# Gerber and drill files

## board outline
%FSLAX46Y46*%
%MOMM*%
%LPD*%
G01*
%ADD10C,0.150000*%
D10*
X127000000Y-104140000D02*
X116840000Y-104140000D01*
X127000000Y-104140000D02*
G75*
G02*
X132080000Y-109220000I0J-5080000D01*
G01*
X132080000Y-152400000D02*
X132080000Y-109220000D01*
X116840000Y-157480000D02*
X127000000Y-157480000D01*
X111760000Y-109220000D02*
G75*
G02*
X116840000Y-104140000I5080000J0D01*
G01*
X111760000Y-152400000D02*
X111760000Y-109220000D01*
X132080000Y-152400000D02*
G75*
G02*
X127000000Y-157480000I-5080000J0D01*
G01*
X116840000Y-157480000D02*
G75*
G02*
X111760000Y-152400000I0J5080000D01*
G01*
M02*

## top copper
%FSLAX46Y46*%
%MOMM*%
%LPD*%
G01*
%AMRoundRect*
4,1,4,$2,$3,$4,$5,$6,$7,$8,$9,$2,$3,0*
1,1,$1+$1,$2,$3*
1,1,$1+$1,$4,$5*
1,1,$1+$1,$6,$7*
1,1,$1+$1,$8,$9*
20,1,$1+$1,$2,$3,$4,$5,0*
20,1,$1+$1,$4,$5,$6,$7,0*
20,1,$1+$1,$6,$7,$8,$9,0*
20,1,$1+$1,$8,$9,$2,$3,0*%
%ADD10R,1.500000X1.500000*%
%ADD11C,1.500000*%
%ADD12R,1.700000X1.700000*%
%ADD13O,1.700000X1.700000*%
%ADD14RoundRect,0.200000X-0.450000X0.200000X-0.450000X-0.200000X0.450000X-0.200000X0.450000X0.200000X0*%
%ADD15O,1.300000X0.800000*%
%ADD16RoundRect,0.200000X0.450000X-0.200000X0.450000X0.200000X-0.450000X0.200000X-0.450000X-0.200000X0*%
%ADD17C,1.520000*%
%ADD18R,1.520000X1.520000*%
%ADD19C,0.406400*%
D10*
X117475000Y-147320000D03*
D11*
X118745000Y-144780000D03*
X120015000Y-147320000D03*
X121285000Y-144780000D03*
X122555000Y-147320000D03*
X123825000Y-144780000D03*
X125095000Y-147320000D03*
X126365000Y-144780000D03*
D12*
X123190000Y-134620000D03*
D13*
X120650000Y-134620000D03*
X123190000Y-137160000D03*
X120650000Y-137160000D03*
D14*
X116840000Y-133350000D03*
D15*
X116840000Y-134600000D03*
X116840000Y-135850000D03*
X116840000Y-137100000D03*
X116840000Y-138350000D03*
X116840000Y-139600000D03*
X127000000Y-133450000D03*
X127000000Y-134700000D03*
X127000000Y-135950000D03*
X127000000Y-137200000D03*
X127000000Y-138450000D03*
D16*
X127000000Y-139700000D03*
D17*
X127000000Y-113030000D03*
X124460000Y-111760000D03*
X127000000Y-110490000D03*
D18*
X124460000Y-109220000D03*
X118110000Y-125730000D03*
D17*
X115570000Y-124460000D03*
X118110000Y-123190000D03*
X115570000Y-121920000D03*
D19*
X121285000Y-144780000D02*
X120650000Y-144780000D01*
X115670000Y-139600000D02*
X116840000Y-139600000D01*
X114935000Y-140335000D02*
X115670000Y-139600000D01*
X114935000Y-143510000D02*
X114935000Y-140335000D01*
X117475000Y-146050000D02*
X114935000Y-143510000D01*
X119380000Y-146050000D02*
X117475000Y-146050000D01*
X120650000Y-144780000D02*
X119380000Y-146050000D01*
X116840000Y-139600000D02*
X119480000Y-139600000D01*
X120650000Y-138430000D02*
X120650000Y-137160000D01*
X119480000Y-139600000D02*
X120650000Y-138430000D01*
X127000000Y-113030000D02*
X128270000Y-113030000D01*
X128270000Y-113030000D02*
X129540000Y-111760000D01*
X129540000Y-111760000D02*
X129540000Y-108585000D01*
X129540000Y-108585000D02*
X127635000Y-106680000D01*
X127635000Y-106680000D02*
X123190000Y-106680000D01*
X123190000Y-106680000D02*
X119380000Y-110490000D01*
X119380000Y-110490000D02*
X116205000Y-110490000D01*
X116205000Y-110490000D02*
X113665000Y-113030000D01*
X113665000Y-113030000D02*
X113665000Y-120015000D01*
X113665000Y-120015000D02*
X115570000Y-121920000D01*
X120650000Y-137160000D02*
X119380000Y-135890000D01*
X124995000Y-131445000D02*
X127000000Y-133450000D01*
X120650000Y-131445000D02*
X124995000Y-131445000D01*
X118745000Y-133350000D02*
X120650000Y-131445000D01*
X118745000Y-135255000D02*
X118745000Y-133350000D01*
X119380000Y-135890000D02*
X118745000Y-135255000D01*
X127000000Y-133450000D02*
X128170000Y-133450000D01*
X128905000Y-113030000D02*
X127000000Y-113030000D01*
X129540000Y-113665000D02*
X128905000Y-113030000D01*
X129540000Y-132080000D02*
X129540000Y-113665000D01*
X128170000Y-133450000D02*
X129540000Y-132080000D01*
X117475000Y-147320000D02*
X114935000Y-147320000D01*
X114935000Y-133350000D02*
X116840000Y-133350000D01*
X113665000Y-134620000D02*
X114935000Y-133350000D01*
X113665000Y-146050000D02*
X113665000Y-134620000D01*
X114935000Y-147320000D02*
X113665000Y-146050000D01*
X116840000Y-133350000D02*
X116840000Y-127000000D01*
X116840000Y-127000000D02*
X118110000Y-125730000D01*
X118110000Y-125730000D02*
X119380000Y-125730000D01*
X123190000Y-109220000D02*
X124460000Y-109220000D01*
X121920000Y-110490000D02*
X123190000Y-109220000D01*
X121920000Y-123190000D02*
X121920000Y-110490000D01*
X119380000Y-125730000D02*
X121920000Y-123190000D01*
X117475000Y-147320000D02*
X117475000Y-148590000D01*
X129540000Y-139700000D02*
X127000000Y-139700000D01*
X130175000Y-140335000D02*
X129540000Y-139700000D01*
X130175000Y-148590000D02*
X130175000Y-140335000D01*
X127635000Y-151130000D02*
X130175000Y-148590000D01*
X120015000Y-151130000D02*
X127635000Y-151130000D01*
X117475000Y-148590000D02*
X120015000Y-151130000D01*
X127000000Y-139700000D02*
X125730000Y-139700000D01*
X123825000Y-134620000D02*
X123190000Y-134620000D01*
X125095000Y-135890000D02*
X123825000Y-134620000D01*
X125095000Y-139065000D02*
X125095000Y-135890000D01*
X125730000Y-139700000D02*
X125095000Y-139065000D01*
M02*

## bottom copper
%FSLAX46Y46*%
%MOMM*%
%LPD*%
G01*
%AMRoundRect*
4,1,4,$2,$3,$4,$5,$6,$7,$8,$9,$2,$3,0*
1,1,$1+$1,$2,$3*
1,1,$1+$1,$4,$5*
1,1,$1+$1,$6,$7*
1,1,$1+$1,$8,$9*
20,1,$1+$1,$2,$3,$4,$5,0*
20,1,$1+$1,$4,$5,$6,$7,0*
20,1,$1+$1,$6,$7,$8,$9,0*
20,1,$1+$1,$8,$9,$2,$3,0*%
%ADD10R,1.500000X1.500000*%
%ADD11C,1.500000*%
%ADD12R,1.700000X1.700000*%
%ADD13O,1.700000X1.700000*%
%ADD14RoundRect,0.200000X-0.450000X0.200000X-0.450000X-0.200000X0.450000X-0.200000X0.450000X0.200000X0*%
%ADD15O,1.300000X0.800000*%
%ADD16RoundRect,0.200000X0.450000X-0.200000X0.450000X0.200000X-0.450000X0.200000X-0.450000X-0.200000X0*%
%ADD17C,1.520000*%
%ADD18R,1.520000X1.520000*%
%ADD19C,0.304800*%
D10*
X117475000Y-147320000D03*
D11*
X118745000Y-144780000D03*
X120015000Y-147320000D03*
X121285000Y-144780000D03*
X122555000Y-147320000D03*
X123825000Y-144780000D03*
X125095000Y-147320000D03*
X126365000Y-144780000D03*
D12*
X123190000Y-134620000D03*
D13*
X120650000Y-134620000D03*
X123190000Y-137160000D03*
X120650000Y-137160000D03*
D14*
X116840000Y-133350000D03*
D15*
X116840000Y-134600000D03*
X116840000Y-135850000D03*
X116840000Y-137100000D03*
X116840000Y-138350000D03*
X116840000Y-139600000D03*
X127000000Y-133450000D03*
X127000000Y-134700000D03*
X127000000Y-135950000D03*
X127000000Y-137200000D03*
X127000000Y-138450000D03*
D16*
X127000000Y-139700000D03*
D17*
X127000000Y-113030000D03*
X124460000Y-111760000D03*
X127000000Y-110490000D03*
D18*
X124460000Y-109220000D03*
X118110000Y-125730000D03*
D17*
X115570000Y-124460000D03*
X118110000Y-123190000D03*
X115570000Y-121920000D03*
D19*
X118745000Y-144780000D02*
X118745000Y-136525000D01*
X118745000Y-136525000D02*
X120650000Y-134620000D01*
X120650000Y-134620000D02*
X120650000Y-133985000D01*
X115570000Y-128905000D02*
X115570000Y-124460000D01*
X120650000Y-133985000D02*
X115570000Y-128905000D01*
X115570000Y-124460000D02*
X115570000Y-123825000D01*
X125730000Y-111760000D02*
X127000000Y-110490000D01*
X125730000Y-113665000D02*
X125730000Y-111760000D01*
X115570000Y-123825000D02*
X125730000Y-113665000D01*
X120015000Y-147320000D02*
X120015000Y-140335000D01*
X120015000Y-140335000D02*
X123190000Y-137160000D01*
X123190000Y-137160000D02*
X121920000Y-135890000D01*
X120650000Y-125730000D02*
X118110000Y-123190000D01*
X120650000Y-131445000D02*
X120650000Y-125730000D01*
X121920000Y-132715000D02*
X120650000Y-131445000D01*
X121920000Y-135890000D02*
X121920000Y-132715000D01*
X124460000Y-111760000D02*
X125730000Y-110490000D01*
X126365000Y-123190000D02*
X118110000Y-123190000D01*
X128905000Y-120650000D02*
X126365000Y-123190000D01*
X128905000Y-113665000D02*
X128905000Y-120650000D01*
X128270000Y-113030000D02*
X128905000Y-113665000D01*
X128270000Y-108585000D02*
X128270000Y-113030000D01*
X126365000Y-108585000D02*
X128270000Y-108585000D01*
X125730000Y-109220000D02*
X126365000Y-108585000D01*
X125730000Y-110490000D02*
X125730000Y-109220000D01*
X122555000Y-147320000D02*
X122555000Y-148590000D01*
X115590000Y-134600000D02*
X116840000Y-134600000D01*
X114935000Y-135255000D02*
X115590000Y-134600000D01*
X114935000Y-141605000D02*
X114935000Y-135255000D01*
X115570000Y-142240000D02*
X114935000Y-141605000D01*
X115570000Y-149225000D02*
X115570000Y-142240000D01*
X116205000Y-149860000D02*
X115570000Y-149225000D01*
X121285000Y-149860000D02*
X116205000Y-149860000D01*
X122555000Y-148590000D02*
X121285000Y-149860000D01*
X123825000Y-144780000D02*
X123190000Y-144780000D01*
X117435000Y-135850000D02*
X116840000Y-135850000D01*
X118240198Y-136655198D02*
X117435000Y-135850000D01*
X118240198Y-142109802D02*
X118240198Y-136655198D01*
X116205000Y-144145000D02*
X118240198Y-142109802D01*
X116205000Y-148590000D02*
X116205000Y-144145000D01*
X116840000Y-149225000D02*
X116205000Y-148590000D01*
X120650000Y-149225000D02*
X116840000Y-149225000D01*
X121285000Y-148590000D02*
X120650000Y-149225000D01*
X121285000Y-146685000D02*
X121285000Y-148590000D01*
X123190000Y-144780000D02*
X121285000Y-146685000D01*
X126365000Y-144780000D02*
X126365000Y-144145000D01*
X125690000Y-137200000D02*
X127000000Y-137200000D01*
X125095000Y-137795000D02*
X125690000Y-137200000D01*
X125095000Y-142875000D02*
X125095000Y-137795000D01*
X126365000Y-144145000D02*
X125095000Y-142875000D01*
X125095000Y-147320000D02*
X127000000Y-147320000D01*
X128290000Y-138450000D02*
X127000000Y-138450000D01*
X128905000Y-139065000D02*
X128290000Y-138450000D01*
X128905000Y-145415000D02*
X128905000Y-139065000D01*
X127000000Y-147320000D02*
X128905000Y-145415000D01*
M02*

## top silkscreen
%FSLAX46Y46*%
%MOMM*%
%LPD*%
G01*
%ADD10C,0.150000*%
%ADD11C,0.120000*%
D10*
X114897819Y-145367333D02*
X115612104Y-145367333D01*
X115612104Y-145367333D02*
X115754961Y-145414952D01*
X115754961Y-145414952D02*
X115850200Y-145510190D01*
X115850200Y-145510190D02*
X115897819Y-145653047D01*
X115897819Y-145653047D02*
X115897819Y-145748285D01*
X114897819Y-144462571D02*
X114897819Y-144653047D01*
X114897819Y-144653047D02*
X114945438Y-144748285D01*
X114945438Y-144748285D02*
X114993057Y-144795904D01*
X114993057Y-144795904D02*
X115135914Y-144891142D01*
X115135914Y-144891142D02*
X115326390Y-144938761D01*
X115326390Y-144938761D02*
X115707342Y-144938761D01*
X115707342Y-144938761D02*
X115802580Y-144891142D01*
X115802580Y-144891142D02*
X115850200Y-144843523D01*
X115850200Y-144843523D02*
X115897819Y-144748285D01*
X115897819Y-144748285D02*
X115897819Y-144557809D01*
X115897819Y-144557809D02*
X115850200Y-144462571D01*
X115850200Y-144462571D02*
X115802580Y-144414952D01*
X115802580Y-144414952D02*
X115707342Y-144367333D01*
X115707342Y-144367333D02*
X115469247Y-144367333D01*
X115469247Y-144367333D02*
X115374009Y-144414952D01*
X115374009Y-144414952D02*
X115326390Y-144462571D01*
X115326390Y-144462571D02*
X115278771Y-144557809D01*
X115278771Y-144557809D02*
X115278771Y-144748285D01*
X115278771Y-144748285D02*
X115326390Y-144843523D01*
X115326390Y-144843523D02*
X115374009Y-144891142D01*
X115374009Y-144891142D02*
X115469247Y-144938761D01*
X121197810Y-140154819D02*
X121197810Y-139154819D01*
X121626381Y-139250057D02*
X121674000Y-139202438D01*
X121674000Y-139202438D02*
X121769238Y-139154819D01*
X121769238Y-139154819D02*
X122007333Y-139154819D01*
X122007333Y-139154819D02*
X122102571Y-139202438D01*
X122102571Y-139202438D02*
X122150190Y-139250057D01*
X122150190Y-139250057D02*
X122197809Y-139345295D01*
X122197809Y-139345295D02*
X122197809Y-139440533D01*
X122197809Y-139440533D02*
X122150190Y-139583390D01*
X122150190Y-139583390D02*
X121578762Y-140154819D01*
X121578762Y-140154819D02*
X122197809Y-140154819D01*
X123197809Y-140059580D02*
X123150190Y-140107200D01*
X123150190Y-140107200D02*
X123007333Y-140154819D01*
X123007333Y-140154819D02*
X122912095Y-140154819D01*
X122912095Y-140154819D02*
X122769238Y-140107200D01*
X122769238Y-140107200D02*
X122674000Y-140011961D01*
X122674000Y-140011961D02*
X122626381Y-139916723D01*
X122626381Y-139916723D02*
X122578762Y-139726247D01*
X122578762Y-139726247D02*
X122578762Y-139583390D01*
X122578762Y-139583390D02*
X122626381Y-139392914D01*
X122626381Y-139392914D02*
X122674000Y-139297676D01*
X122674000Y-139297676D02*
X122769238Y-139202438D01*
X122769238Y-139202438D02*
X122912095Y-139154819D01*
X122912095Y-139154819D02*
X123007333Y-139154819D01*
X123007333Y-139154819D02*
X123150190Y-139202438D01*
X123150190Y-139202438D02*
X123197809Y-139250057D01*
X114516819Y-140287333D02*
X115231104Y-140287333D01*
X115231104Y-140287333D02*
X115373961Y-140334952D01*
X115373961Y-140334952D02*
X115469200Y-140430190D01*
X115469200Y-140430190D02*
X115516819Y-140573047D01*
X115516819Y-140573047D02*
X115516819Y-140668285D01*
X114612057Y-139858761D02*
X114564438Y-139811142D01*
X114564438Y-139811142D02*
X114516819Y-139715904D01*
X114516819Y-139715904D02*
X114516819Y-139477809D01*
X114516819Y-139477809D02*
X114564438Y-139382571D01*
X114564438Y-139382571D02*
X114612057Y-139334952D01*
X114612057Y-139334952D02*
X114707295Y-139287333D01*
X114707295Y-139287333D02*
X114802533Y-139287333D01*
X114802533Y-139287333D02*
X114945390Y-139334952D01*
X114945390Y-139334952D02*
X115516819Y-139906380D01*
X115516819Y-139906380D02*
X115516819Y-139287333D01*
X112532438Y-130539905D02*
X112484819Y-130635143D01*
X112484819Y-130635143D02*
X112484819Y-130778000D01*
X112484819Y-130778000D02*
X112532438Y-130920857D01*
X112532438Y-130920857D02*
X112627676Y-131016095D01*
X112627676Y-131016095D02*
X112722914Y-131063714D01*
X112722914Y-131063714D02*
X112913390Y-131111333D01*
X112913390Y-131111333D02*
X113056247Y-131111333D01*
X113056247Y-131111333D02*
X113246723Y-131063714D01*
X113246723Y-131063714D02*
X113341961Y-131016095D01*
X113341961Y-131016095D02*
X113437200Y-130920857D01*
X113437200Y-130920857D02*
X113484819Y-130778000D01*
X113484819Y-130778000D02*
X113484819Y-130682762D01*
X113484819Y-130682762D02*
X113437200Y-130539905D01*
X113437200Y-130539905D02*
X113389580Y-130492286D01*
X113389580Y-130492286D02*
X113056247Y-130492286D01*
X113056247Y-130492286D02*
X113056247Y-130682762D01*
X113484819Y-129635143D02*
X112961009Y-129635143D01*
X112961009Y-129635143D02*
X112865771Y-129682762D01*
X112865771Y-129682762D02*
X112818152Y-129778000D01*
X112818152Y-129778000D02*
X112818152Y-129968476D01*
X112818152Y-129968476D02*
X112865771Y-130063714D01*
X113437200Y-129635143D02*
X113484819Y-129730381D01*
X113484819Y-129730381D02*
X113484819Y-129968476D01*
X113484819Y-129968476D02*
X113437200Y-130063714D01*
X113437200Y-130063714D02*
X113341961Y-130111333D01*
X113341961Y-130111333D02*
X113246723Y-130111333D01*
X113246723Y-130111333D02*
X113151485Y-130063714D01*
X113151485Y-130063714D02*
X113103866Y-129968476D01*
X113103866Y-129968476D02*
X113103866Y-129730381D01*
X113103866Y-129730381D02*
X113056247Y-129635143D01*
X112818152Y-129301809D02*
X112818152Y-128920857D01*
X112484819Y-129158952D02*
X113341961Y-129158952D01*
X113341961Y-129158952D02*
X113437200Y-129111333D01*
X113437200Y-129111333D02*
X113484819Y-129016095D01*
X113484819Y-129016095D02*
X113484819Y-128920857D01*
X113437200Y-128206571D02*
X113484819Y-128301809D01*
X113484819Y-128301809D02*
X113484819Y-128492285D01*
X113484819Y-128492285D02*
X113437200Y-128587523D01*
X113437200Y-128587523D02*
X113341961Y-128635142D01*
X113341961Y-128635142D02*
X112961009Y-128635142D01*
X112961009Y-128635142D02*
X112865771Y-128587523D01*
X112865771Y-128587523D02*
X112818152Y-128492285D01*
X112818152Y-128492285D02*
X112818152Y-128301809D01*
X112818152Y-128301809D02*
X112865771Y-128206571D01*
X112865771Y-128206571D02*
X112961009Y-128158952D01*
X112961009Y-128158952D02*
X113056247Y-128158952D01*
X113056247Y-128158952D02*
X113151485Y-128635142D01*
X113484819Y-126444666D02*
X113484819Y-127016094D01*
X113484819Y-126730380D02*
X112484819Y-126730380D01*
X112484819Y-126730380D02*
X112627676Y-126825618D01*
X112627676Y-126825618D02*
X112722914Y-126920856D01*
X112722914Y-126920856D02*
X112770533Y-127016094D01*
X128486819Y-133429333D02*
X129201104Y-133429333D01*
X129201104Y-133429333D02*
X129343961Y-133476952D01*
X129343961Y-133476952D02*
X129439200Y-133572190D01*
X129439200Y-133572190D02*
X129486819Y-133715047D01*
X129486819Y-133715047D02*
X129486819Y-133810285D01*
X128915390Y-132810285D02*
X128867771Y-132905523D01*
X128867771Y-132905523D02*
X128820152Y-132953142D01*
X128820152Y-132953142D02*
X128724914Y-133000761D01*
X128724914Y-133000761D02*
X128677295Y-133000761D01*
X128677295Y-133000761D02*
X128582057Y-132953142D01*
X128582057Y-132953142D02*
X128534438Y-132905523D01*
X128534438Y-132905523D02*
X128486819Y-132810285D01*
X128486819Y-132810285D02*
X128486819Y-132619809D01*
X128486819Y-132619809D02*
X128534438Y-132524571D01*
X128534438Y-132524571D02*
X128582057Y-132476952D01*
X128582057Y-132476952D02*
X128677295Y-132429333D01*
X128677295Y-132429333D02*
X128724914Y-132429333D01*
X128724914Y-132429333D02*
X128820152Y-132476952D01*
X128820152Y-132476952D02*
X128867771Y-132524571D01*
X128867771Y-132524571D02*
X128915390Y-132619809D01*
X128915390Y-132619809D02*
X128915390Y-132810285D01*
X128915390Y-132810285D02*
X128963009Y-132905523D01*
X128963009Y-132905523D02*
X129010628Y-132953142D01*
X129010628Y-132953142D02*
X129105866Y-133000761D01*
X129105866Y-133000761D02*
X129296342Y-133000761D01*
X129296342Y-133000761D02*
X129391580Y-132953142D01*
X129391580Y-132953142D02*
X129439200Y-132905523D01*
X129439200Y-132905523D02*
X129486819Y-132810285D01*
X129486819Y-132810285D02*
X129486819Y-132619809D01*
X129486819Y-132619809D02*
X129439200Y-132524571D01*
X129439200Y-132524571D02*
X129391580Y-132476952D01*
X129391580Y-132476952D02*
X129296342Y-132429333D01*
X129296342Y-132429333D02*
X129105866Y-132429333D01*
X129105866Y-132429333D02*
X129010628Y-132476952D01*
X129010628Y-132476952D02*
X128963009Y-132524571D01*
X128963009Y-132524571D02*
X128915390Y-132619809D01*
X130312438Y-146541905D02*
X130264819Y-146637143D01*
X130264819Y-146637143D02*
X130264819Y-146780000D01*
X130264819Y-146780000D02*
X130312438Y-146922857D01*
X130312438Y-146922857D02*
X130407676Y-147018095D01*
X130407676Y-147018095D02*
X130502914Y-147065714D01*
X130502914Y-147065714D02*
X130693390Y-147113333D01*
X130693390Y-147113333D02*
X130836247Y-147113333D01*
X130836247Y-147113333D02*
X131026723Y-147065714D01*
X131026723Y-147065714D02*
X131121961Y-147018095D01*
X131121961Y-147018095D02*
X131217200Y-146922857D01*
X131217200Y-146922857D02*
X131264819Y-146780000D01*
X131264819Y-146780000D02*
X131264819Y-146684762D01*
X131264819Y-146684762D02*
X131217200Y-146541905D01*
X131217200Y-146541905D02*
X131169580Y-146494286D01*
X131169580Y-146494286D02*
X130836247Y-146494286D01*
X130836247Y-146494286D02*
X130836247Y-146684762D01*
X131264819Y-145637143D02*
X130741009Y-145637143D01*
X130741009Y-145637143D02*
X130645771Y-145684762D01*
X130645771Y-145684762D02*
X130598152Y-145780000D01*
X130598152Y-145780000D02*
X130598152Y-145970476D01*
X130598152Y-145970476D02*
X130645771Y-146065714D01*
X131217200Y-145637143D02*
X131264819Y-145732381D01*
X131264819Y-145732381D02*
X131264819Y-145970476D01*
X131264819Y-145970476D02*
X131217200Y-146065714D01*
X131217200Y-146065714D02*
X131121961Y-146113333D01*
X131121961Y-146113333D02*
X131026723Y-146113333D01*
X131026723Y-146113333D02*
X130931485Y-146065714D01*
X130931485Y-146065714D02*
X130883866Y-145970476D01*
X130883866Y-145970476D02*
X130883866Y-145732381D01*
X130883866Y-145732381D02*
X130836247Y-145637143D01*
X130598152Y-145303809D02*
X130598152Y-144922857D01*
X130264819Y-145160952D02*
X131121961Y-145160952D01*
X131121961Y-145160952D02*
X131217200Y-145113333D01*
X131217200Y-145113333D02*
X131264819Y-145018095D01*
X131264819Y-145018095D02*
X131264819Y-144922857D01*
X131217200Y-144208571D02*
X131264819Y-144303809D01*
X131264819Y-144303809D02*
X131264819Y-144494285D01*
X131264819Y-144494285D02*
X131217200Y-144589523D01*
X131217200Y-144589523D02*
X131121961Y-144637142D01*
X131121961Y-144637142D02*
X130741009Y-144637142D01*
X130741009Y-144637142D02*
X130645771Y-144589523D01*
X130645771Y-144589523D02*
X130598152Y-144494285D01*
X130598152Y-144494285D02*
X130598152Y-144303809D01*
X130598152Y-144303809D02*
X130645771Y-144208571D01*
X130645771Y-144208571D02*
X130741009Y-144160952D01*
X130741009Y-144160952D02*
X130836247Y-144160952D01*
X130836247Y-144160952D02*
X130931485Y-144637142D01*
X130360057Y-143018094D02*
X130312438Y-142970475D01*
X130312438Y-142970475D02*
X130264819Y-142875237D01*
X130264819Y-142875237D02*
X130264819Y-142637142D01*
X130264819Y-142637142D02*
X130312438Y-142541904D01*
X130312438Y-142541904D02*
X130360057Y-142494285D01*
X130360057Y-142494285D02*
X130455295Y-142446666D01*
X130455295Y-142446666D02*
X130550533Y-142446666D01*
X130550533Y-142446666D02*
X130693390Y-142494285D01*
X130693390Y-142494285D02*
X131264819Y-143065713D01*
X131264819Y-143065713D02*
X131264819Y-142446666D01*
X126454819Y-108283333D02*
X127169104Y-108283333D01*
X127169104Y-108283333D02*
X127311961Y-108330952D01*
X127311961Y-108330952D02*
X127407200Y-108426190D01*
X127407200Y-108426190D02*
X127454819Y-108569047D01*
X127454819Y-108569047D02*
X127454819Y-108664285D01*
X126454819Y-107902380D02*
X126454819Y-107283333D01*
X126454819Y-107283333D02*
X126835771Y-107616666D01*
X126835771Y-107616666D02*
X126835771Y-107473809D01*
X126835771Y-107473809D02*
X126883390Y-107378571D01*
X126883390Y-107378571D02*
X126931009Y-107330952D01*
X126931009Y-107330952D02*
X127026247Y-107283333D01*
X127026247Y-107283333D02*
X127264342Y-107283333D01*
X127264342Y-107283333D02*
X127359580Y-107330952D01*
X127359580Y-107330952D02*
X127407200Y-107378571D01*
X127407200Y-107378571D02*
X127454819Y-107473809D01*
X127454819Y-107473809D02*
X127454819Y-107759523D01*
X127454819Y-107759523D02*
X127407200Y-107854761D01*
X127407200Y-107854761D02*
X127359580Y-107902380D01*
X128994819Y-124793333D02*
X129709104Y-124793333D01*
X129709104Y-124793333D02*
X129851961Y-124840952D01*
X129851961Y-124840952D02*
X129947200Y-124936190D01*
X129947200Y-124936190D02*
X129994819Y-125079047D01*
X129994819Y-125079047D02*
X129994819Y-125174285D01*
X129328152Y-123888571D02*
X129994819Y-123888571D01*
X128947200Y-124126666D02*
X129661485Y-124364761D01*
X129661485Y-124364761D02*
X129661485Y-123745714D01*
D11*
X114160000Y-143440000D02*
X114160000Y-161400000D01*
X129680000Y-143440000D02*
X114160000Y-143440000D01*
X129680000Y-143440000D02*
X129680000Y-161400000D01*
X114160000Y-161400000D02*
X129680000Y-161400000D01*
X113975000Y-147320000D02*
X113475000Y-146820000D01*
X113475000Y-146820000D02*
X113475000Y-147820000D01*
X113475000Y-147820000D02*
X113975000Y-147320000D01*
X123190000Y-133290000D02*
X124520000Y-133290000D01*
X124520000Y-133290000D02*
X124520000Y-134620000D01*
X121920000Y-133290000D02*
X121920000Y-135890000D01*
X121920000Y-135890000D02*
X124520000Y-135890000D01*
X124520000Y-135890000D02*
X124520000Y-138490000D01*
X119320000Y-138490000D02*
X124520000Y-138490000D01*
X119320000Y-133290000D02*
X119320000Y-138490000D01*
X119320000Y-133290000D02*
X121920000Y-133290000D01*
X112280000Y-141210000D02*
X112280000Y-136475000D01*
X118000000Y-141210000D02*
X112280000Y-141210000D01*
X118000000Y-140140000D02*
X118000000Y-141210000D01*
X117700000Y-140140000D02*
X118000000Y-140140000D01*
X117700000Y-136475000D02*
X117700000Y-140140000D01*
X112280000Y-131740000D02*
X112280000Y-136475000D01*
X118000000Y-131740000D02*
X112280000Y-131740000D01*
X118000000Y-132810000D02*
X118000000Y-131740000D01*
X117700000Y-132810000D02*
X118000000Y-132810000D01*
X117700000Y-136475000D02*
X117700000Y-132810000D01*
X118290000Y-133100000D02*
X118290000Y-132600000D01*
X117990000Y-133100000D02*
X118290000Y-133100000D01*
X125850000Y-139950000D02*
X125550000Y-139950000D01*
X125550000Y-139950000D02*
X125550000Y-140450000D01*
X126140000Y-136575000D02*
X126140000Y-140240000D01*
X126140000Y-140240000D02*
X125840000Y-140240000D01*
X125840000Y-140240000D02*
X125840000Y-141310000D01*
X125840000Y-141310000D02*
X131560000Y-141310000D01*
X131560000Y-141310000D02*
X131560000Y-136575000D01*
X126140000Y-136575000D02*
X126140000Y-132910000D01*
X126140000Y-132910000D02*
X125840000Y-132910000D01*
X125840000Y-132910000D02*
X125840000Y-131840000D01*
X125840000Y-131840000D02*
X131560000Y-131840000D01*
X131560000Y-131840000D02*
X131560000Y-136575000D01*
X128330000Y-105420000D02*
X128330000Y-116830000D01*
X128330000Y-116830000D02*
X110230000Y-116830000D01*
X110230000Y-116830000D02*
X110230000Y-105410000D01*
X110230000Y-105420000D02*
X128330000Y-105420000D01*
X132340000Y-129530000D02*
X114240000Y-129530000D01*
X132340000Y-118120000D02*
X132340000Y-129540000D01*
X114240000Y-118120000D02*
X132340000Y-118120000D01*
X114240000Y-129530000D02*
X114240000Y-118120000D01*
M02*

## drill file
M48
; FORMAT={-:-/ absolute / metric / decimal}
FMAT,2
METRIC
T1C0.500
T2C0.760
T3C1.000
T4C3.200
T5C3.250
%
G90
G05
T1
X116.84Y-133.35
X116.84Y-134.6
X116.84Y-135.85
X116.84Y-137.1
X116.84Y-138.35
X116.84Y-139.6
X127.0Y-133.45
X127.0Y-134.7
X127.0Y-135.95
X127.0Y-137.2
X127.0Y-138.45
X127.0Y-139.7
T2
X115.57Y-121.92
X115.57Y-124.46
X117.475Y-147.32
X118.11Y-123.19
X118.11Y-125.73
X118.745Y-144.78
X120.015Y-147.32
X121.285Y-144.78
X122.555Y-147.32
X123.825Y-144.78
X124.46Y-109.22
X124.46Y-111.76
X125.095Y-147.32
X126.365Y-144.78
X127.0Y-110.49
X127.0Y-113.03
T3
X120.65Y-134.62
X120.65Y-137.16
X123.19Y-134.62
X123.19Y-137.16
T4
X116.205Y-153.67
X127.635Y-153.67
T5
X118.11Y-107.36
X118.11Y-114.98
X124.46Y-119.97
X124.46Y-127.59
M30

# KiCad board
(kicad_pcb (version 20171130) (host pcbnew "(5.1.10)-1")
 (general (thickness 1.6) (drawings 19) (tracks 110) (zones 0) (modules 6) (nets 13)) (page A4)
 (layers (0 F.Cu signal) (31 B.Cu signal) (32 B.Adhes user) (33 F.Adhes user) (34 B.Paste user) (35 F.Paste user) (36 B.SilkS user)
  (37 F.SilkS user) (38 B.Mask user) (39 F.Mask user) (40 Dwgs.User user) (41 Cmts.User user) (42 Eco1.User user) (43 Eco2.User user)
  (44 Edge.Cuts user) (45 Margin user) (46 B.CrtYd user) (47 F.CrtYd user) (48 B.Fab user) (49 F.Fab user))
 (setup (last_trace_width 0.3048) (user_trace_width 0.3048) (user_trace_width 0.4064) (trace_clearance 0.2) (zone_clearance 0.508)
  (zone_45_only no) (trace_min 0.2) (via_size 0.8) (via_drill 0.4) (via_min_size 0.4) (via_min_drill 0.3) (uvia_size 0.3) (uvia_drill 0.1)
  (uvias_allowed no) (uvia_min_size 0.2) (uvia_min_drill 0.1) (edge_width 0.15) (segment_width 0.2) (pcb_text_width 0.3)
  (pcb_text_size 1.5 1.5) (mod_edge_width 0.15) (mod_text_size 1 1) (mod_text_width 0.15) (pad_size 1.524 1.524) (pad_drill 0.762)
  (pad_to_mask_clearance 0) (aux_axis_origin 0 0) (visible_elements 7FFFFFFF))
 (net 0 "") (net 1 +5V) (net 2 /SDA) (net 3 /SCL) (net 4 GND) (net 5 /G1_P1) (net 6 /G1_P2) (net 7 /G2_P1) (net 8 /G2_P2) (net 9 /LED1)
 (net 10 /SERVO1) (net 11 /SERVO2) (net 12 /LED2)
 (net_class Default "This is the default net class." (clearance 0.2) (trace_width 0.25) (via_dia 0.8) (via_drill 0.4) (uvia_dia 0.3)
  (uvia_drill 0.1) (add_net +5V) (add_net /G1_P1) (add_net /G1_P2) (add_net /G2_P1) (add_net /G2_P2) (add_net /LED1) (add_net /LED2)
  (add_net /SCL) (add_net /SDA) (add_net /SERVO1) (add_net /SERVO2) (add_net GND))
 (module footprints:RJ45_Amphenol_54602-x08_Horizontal (layer F.Cu) (at 117.475 147.32)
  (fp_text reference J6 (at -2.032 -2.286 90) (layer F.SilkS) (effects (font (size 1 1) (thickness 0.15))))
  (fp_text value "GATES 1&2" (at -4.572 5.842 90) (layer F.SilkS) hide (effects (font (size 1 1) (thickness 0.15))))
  (fp_line (start -3.315 -3.88) (end -3.315 14.08) (layer F.SilkS) (width 0.12))
  (fp_line (start 12.205 -3.88) (end -3.315 -3.88) (layer F.SilkS) (width 0.12))
  (fp_line (start 12.205 -3.88) (end 12.205 14.08) (layer F.SilkS) (width 0.12))
  (fp_line (start -3.315 14.08) (end 12.205 14.08) (layer F.SilkS) (width 0.12))
  (fp_line (start -3.5 0) (end -4 -0.5) (layer F.SilkS) (width 0.12))
  (fp_line (start -4 -0.5) (end -4 0.5) (layer F.SilkS) (width 0.12))
  (fp_line (start -4 0.5) (end -3.5 0) (layer F.SilkS) (width 0.12))
  (pad "" np_thru_hole circle (at 10.16 6.35) (size 3.2 3.2) (drill 3.2) (layers *.Cu *.Mask))
  (pad "" np_thru_hole circle (at -1.27 6.35) (size 3.2 3.2) (drill 3.2) (layers *.Cu *.Mask))
  (pad 1 thru_hole rect (at 0 0) (size 1.5 1.5) (drill 0.76) (layers *.Cu *.Mask) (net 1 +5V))
  (pad 2 thru_hole circle (at 1.27 -2.54) (size 1.5 1.5) (drill 0.76) (layers *.Cu *.Mask) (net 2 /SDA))
  (pad 3 thru_hole circle (at 2.54 0) (size 1.5 1.5) (drill 0.76) (layers *.Cu *.Mask) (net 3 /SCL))
  (pad 4 thru_hole circle (at 3.81 -2.54) (size 1.5 1.5) (drill 0.76) (layers *.Cu *.Mask) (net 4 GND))
  (pad 5 thru_hole circle (at 5.08 0) (size 1.5 1.5) (drill 0.76) (layers *.Cu *.Mask) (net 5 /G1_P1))
  (pad 6 thru_hole circle (at 6.35 -2.54) (size 1.5 1.5) (drill 0.76) (layers *.Cu *.Mask) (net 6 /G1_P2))
  (pad 7 thru_hole circle (at 7.62 0) (size 1.5 1.5) (drill 0.76) (layers *.Cu *.Mask) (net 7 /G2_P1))
  (pad 8 thru_hole circle (at 8.89 -2.54) (size 1.5 1.5) (drill 0.76) (layers *.Cu *.Mask) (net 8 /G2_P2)))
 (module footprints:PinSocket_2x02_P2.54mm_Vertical (layer F.Cu) (at 123.19 134.62)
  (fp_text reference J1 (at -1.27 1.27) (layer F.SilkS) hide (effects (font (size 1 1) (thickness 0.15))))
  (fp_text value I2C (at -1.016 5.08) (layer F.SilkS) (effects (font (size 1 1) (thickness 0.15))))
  (fp_line (start 0 -1.33) (end 1.33 -1.33) (layer F.SilkS) (width 0.12))
  (fp_line (start 1.33 -1.33) (end 1.33 0) (layer F.SilkS) (width 0.12))
  (fp_line (start -1.27 -1.33) (end -1.27 1.27) (layer F.SilkS) (width 0.12))
  (fp_line (start -1.27 1.27) (end 1.33 1.27) (layer F.SilkS) (width 0.12))
  (fp_line (start 1.33 1.27) (end 1.33 3.87) (layer F.SilkS) (width 0.12))
  (fp_line (start -3.87 3.87) (end 1.33 3.87) (layer F.SilkS) (width 0.12))
  (fp_line (start -3.87 -1.33) (end -3.87 3.87) (layer F.SilkS) (width 0.12))
  (fp_line (start -3.87 -1.33) (end -1.27 -1.33) (layer F.SilkS) (width 0.12))
  (pad 1 thru_hole rect (at 0 0) (size 1.7 1.7) (drill 1) (layers *.Cu *.Mask) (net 1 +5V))
  (pad 2 thru_hole oval (at -2.54 0) (size 1.7 1.7) (drill 1) (layers *.Cu *.Mask) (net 2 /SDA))
  (pad 3 thru_hole oval (at 0 2.54) (size 1.7 1.7) (drill 1) (layers *.Cu *.Mask) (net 3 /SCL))
  (pad 4 thru_hole oval (at -2.54 2.54) (size 1.7 1.7) (drill 1) (layers *.Cu *.Mask) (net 4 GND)))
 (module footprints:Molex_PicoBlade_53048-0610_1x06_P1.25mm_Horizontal (layer F.Cu) (at 116.84 133.35 270)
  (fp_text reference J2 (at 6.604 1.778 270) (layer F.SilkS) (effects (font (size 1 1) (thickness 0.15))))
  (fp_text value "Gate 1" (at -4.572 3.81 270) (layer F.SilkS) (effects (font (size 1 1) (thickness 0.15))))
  (fp_line (start 7.86 4.56) (end 3.125 4.56) (layer F.SilkS) (width 0.12))
  (fp_line (start 7.86 -1.16) (end 7.86 4.56) (layer F.SilkS) (width 0.12))
  (fp_line (start 6.79 -1.16) (end 7.86 -1.16) (layer F.SilkS) (width 0.12))
  (fp_line (start 6.79 -0.86) (end 6.79 -1.16) (layer F.SilkS) (width 0.12))
  (fp_line (start 3.125 -0.86) (end 6.79 -0.86) (layer F.SilkS) (width 0.12))
  (fp_line (start -1.61 4.56) (end 3.125 4.56) (layer F.SilkS) (width 0.12))
  (fp_line (start -1.61 -1.16) (end -1.61 4.56) (layer F.SilkS) (width 0.12))
  (fp_line (start -0.54 -1.16) (end -1.61 -1.16) (layer F.SilkS) (width 0.12))
  (fp_line (start -0.54 -0.86) (end -0.54 -1.16) (layer F.SilkS) (width 0.12))
  (fp_line (start 3.125 -0.86) (end -0.54 -0.86) (layer F.SilkS) (width 0.12))
  (fp_line (start -0.25 -1.45) (end -0.75 -1.45) (layer F.SilkS) (width 0.12))
  (fp_line (start -0.25 -1.15) (end -0.25 -1.45) (layer F.SilkS) (width 0.12))
  (pad 1 thru_hole roundrect (at 0 0 270) (size 0.8 1.3) (drill 0.5) (layers *.Cu *.Mask) (roundrect_rratio 0.25) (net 1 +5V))
  (pad 2 thru_hole oval (at 1.25 0 270) (size 0.8 1.3) (drill 0.5) (layers *.Cu *.Mask) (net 5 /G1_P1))
  (pad 3 thru_hole oval (at 2.5 0 270) (size 0.8 1.3) (drill 0.5) (layers *.Cu *.Mask) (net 6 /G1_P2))
  (pad 4 thru_hole oval (at 3.75 0 270) (size 0.8 1.3) (drill 0.5) (layers *.Cu *.Mask) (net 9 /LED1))
  (pad 5 thru_hole oval (at 5 0 270) (size 0.8 1.3) (drill 0.5) (layers *.Cu *.Mask) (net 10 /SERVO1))
  (pad 6 thru_hole oval (at 6.25 0 270) (size 0.8 1.3) (drill 0.5) (layers *.Cu *.Mask) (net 4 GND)))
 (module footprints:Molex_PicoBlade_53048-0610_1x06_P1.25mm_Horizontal (layer F.Cu) (at 127 139.7 90)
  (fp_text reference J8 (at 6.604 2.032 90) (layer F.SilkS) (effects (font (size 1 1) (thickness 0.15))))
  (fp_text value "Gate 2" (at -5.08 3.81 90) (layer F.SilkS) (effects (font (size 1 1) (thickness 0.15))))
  (fp_line (start -0.25 -1.15) (end -0.25 -1.45) (layer F.SilkS) (width 0.12))
  (fp_line (start -0.25 -1.45) (end -0.75 -1.45) (layer F.SilkS) (width 0.12))
  (fp_line (start 3.125 -0.86) (end -0.54 -0.86) (layer F.SilkS) (width 0.12))
  (fp_line (start -0.54 -0.86) (end -0.54 -1.16) (layer F.SilkS) (width 0.12))
  (fp_line (start -0.54 -1.16) (end -1.61 -1.16) (layer F.SilkS) (width 0.12))
  (fp_line (start -1.61 -1.16) (end -1.61 4.56) (layer F.SilkS) (width 0.12))
  (fp_line (start -1.61 4.56) (end 3.125 4.56) (layer F.SilkS) (width 0.12))
  (fp_line (start 3.125 -0.86) (end 6.79 -0.86) (layer F.SilkS) (width 0.12))
  (fp_line (start 6.79 -0.86) (end 6.79 -1.16) (layer F.SilkS) (width 0.12))
  (fp_line (start 6.79 -1.16) (end 7.86 -1.16) (layer F.SilkS) (width 0.12))
  (fp_line (start 7.86 -1.16) (end 7.86 4.56) (layer F.SilkS) (width 0.12))
  (fp_line (start 7.86 4.56) (end 3.125 4.56) (layer F.SilkS) (width 0.12))
  (pad 6 thru_hole oval (at 6.25 0 90) (size 0.8 1.3) (drill 0.5) (layers *.Cu *.Mask) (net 4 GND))
  (pad 5 thru_hole oval (at 5 0 90) (size 0.8 1.3) (drill 0.5) (layers *.Cu *.Mask) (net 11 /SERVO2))
  (pad 4 thru_hole oval (at 3.75 0 90) (size 0.8 1.3) (drill 0.5) (layers *.Cu *.Mask) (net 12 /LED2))
  (pad 3 thru_hole oval (at 2.5 0 90) (size 0.8 1.3) (drill 0.5) (layers *.Cu *.Mask) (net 8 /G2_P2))
  (pad 2 thru_hole oval (at 1.25 0 90) (size 0.8 1.3) (drill 0.5) (layers *.Cu *.Mask) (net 7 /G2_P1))
  (pad 1 thru_hole roundrect (at 0 0 90) (size 0.8 1.3) (drill 0.5) (layers *.Cu *.Mask) (roundrect_rratio 0.25) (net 1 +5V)))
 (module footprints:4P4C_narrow (layer F.Cu) (at 127 109.22 270)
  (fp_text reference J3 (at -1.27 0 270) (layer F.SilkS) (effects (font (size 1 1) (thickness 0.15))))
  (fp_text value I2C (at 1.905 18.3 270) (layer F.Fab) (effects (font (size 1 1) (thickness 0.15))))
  (fp_line (start -3.8 -1.33) (end 7.61 -1.33) (layer F.SilkS) (width 0.12))
  (fp_line (start 7.61 -1.33) (end 7.61 16.77) (layer F.SilkS) (width 0.12))
  (fp_line (start 7.61 16.77) (end -3.81 16.77) (layer F.SilkS) (width 0.12))
  (fp_line (start -3.8 16.77) (end -3.8 -1.33) (layer F.SilkS) (width 0.12))
  (pad "" np_thru_hole circle (at 5.76 8.89 270) (size 3.25 3.25) (drill 3.25) (layers *.Cu *.Mask))
  (pad 4 thru_hole circle (at 3.81 0 270) (size 1.52 1.52) (drill 0.76) (layers *.Cu *.Mask) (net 4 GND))
  (pad 3 thru_hole circle (at 2.54 2.54 270) (size 1.52 1.52) (drill 0.76) (layers *.Cu *.Mask) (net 3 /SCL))
  (pad 2 thru_hole circle (at 1.27 0 270) (size 1.52 1.52) (drill 0.76) (layers *.Cu *.Mask) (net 2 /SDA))
  (pad "" np_thru_hole circle (at -1.86 8.89 270) (size 3.25 3.25) (drill 3.25) (layers *.Cu *.Mask))
  (pad 1 thru_hole rect (at 0 2.54 270) (size 1.52 1.52) (drill 0.76) (layers *.Cu *.Mask) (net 1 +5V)))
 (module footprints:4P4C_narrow (layer F.Cu) (at 115.57 125.73 90)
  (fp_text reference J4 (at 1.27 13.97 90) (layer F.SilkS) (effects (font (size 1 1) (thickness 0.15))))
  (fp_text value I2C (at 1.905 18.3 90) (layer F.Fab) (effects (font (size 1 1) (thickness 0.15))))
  (fp_line (start -3.8 16.77) (end -3.8 -1.33) (layer F.SilkS) (width 0.12))
  (fp_line (start 7.61 16.77) (end -3.81 16.77) (layer F.SilkS) (width 0.12))
  (fp_line (start 7.61 -1.33) (end 7.61 16.77) (layer F.SilkS) (width 0.12))
  (fp_line (start -3.8 -1.33) (end 7.61 -1.33) (layer F.SilkS) (width 0.12))
  (pad 1 thru_hole rect (at 0 2.54 90) (size 1.52 1.52) (drill 0.76) (layers *.Cu *.Mask) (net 1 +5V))
  (pad "" np_thru_hole circle (at -1.86 8.89 90) (size 3.25 3.25) (drill 3.25) (layers *.Cu *.Mask))
  (pad 2 thru_hole circle (at 1.27 0 90) (size 1.52 1.52) (drill 0.76) (layers *.Cu *.Mask) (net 2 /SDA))
  (pad 3 thru_hole circle (at 2.54 2.54 90) (size 1.52 1.52) (drill 0.76) (layers *.Cu *.Mask) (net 3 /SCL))
  (pad 4 thru_hole circle (at 3.81 0 90) (size 1.52 1.52) (drill 0.76) (layers *.Cu *.Mask) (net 4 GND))
  (pad "" np_thru_hole circle (at 5.76 8.89 90) (size 3.25 3.25) (drill 3.25) (layers *.Cu *.Mask)))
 (gr_line (start 127 104.14) (end 116.84 104.14) (angle 90) (layer Edge.Cuts) (width 0.15))
 (gr_arc (start 127 109.22) (end 127 104.14) (angle 90) (layer Edge.Cuts) (width 0.15))
 (gr_line (start 132.08 152.4) (end 132.08 109.22) (angle 90) (layer Edge.Cuts) (width 0.15))
 (gr_line (start 116.84 157.48) (end 127 157.48) (angle 90) (layer Edge.Cuts) (width 0.15))
 (gr_arc (start 116.84 109.22) (end 111.76 109.22) (angle 90) (layer Edge.Cuts) (width 0.15))
 (gr_line (start 111.76 152.4) (end 111.76 109.22) (angle 90) (layer Edge.Cuts) (width 0.15))
 (gr_arc (start 127 152.4) (end 132.08 152.4) (angle 90) (layer Edge.Cuts) (width 0.15))
 (gr_arc (start 116.84 152.4) (end 116.84 157.48) (angle 90) (layer Edge.Cuts) (width 0.15))
 (segment (start 121.285 144.78) (end 120.65 144.78) (width 0.4064) (layer F.Cu) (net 4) (status C00000))
 (segment (start 115.67 139.6) (end 116.84 139.6) (width 0.4064) (layer F.Cu) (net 4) (status 800000))
 (segment (start 114.935 140.335) (end 115.67 139.6) (width 0.4064) (layer F.Cu) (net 4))
 (segment (start 114.935 143.51) (end 114.935 140.335) (width 0.4064) (layer F.Cu) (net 4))
 (segment (start 117.475 146.05) (end 114.935 143.51) (width 0.4064) (layer F.Cu) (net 4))
 (segment (start 119.38 146.05) (end 117.475 146.05) (width 0.4064) (layer F.Cu) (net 4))
 (segment (start 120.65 144.78) (end 119.38 146.05) (width 0.4064) (layer F.Cu) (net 4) (status 400000))
 (segment (start 116.84 139.6) (end 119.48 139.6) (width 0.4064) (layer F.Cu) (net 4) (status 400000))
 (segment (start 120.65 138.43) (end 120.65 137.16) (width 0.4064) (layer F.Cu) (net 4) (status 800000))
 (segment (start 119.48 139.6) (end 120.65 138.43) (width 0.4064) (layer F.Cu) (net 4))
 (segment (start 127 113.03) (end 128.27 113.03) (width 0.4064) (layer F.Cu) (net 4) (status 400000))
 (segment (start 128.27 113.03) (end 129.54 111.76) (width 0.4064) (layer F.Cu) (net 4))
 (segment (start 129.54 111.76) (end 129.54 108.585) (width 0.4064) (layer F.Cu) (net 4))
 (segment (start 129.54 108.585) (end 127.635 106.68) (width 0.4064) (layer F.Cu) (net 4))
 (segment (start 127.635 106.68) (end 123.19 106.68) (width 0.4064) (layer F.Cu) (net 4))
 (segment (start 123.19 106.68) (end 119.38 110.49) (width 0.4064) (layer F.Cu) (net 4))
 (segment (start 119.38 110.49) (end 116.205 110.49) (width 0.4064) (layer F.Cu) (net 4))
 (segment (start 116.205 110.49) (end 113.665 113.03) (width 0.4064) (layer F.Cu) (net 4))
 (segment (start 113.665 113.03) (end 113.665 120.015) (width 0.4064) (layer F.Cu) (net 4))
 (segment (start 113.665 120.015) (end 115.57 121.92) (width 0.4064) (layer F.Cu) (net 4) (status 800000))
 (segment (start 120.65 137.16) (end 119.38 135.89) (width 0.4064) (layer F.Cu) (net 4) (status 400000))
 (segment (start 124.995 131.445) (end 127 133.45) (width 0.4064) (layer F.Cu) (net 4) (status 800000))
 (segment (start 120.65 131.445) (end 124.995 131.445) (width 0.4064) (layer F.Cu) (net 4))
 (segment (start 118.745 133.35) (end 120.65 131.445) (width 0.4064) (layer F.Cu) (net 4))
 (segment (start 118.745 135.255) (end 118.745 133.35) (width 0.4064) (layer F.Cu) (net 4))
 (segment (start 119.38 135.89) (end 118.745 135.255) (width 0.4064) (layer F.Cu) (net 4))
 (segment (start 127 133.45) (end 128.17 133.45) (width 0.4064) (layer F.Cu) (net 4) (status 400000))
 (segment (start 128.905 113.03) (end 127 113.03) (width 0.4064) (layer F.Cu) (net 4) (status 800000))
 (segment (start 129.54 113.665) (end 128.905 113.03) (width 0.4064) (layer F.Cu) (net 4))
 (segment (start 129.54 132.08) (end 129.54 113.665) (width 0.4064) (layer F.Cu) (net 4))
 (segment (start 128.17 133.45) (end 129.54 132.08) (width 0.4064) (layer F.Cu) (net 4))
 (segment (start 118.745 144.78) (end 118.745 136.525) (width 0.3048) (layer B.Cu) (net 2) (status 400000))
 (segment (start 118.745 136.525) (end 120.65 134.62) (width 0.3048) (layer B.Cu) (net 2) (status 800000))
 (segment (start 120.65 134.62) (end 120.65 133.985) (width 0.3048) (layer B.Cu) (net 2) (status C00000))
 (segment (start 115.57 128.905) (end 115.57 124.46) (width 0.3048) (layer B.Cu) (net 2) (status 800000))
 (segment (start 120.65 133.985) (end 115.57 128.905) (width 0.3048) (layer B.Cu) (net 2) (status 400000))
 (segment (start 115.57 124.46) (end 115.57 123.825) (width 0.3048) (layer B.Cu) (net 2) (status C00000))
 (segment (start 125.73 111.76) (end 127 110.49) (width 0.3048) (layer B.Cu) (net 2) (status 800000))
 (segment (start 125.73 113.665) (end 125.73 111.76) (width 0.3048) (layer B.Cu) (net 2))
 (segment (start 115.57 123.825) (end 125.73 113.665) (width 0.3048) (layer B.Cu) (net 2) (status 400000))
 (segment (start 120.015 147.32) (end 120.015 140.335) (width 0.3048) (layer B.Cu) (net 3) (status 400000))
 (segment (start 120.015 140.335) (end 123.19 137.16) (width 0.3048) (layer B.Cu) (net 3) (status 800000))
 (segment (start 123.19 137.16) (end 121.92 135.89) (width 0.3048) (layer B.Cu) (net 3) (status 400000))
 (segment (start 120.65 125.73) (end 118.11 123.19) (width 0.3048) (layer B.Cu) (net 3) (status 800000))
 (segment (start 120.65 131.445) (end 120.65 125.73) (width 0.3048) (layer B.Cu) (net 3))
 (segment (start 121.92 132.715) (end 120.65 131.445) (width 0.3048) (layer B.Cu) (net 3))
 (segment (start 121.92 135.89) (end 121.92 132.715) (width 0.3048) (layer B.Cu) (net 3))
 (segment (start 124.46 111.76) (end 125.73 110.49) (width 0.3048) (layer B.Cu) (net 3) (status 400000))
 (segment (start 126.365 123.19) (end 118.11 123.19) (width 0.3048) (layer B.Cu) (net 3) (status 800000))
 (segment (start 128.905 120.65) (end 126.365 123.19) (width 0.3048) (layer B.Cu) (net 3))
 (segment (start 128.905 113.665) (end 128.905 120.65) (width 0.3048) (layer B.Cu) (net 3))
 (segment (start 128.27 113.03) (end 128.905 113.665) (width 0.3048) (layer B.Cu) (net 3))
 (segment (start 128.27 108.585) (end 128.27 113.03) (width 0.3048) (layer B.Cu) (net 3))
 (segment (start 126.365 108.585) (end 128.27 108.585) (width 0.3048) (layer B.Cu) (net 3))
 (segment (start 125.73 109.22) (end 126.365 108.585) (width 0.3048) (layer B.Cu) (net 3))
 (segment (start 125.73 110.49) (end 125.73 109.22) (width 0.3048) (layer B.Cu) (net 3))
 (segment (start 117.475 147.32) (end 114.935 147.32) (width 0.4064) (layer F.Cu) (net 1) (status 400000))
 (segment (start 114.935 133.35) (end 116.84 133.35) (width 0.4064) (layer F.Cu) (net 1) (status 800000))
 (segment (start 113.665 134.62) (end 114.935 133.35) (width 0.4064) (layer F.Cu) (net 1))
 (segment (start 113.665 146.05) (end 113.665 134.62) (width 0.4064) (layer F.Cu) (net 1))
 (segment (start 114.935 147.32) (end 113.665 146.05) (width 0.4064) (layer F.Cu) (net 1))
 (segment (start 116.84 133.35) (end 116.84 127) (width 0.4064) (layer F.Cu) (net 1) (status 400000))
 (segment (start 116.84 127) (end 118.11 125.73) (width 0.4064) (layer F.Cu) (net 1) (status 800000))
 (segment (start 118.11 125.73) (end 119.38 125.73) (width 0.4064) (layer F.Cu) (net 1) (status 400000))
 (segment (start 123.19 109.22) (end 124.46 109.22) (width 0.4064) (layer F.Cu) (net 1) (status 800000))
 (segment (start 121.92 110.49) (end 123.19 109.22) (width 0.4064) (layer F.Cu) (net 1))
 (segment (start 121.92 123.19) (end 121.92 110.49) (width 0.4064) (layer F.Cu) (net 1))
 (segment (start 119.38 125.73) (end 121.92 123.19) (width 0.4064) (layer F.Cu) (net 1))
 (segment (start 117.475 147.32) (end 117.475 148.59) (width 0.4064) (layer F.Cu) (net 1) (status 400000))
 (segment (start 129.54 139.7) (end 127 139.7) (width 0.4064) (layer F.Cu) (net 1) (status 800000))
 (segment (start 130.175 140.335) (end 129.54 139.7) (width 0.4064) (layer F.Cu) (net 1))
 (segment (start 130.175 148.59) (end 130.175 140.335) (width 0.4064) (layer F.Cu) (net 1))
 (segment (start 127.635 151.13) (end 130.175 148.59) (width 0.4064) (layer F.Cu) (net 1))
 (segment (start 120.015 151.13) (end 127.635 151.13) (width 0.4064) (layer F.Cu) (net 1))
 (segment (start 117.475 148.59) (end 120.015 151.13) (width 0.4064) (layer F.Cu) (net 1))
 (segment (start 127 139.7) (end 125.73 139.7) (width 0.4064) (layer F.Cu) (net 1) (status 400000))
 (segment (start 123.825 134.62) (end 123.19 134.62) (width 0.4064) (layer F.Cu) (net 1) (status C00000))
 (segment (start 125.095 135.89) (end 123.825 134.62) (width 0.4064) (layer F.Cu) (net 1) (status 800000))
 (segment (start 125.095 139.065) (end 125.095 135.89) (width 0.4064) (layer F.Cu) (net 1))
 (segment (start 125.73 139.7) (end 125.095 139.065) (width 0.4064) (layer F.Cu) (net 1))
 (segment (start 122.555 147.32) (end 122.555 148.59) (width 0.3048) (layer B.Cu) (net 5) (status 400000))
 (segment (start 115.59 134.6) (end 116.84 134.6) (width 0.3048) (layer B.Cu) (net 5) (status 800000))
 (segment (start 114.935 135.255) (end 115.59 134.6) (width 0.3048) (layer B.Cu) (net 5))
 (segment (start 114.935 141.605) (end 114.935 135.255) (width 0.3048) (layer B.Cu) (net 5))
 (segment (start 115.57 142.24) (end 114.935 141.605) (width 0.3048) (layer B.Cu) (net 5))
 (segment (start 115.57 149.225) (end 115.57 142.24) (width 0.3048) (layer B.Cu) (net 5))
 (segment (start 116.205 149.86) (end 115.57 149.225) (width 0.3048) (layer B.Cu) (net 5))
 (segment (start 121.285 149.86) (end 116.205 149.86) (width 0.3048) (layer B.Cu) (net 5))
 (segment (start 122.555 148.59) (end 121.285 149.86) (width 0.3048) (layer B.Cu) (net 5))
 (segment (start 123.825 144.78) (end 123.19 144.78) (width 0.3048) (layer B.Cu) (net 6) (status C00000))
 (segment (start 117.435 135.85) (end 116.84 135.85) (width 0.3048) (layer B.Cu) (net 6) (status C00000))
 (segment (start 118.240198 136.655198) (end 117.435 135.85) (width 0.3048) (layer B.Cu) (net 6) (status 800000))
 (segment (start 118.240198 142.109802) (end 118.240198 136.655198) (width 0.3048) (layer B.Cu) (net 6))
 (segment (start 116.205 144.145) (end 118.240198 142.109802) (width 0.3048) (layer B.Cu) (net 6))
 (segment (start 116.205 148.59) (end 116.205 144.145) (width 0.3048) (layer B.Cu) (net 6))
 (segment (start 116.84 149.225) (end 116.205 148.59) (width 0.3048) (layer B.Cu) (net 6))
 (segment (start 120.65 149.225) (end 116.84 149.225) (width 0.3048) (layer B.Cu) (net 6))
 (segment (start 121.285 148.59) (end 120.65 149.225) (width 0.3048) (layer B.Cu) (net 6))
 (segment (start 121.285 146.685) (end 121.285 148.59) (width 0.3048) (layer B.Cu) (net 6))
 (segment (start 123.19 144.78) (end 121.285 146.685) (width 0.3048) (layer B.Cu) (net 6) (status 400000))
 (segment (start 126.365 144.78) (end 126.365 144.145) (width 0.3048) (layer B.Cu) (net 8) (status C00000))
 (segment (start 125.69 137.2) (end 127 137.2) (width 0.3048) (layer B.Cu) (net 8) (status 800000))
 (segment (start 125.095 137.795) (end 125.69 137.2) (width 0.3048) (layer B.Cu) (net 8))
 (segment (start 125.095 142.875) (end 125.095 137.795) (width 0.3048) (layer B.Cu) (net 8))
 (segment (start 126.365 144.145) (end 125.095 142.875) (width 0.3048) (layer B.Cu) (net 8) (status 400000))
 (segment (start 125.095 147.32) (end 127 147.32) (width 0.3048) (layer B.Cu) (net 7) (status 400000))
 (segment (start 128.29 138.45) (end 127 138.45) (width 0.3048) (layer B.Cu) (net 7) (status 800000))
 (segment (start 128.905 139.065) (end 128.29 138.45) (width 0.3048) (layer B.Cu) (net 7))
 (segment (start 128.905 145.415) (end 128.905 139.065) (width 0.3048) (layer B.Cu) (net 7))
 (segment (start 127 147.32) (end 128.905 145.415) (width 0.3048) (layer B.Cu) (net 7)))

